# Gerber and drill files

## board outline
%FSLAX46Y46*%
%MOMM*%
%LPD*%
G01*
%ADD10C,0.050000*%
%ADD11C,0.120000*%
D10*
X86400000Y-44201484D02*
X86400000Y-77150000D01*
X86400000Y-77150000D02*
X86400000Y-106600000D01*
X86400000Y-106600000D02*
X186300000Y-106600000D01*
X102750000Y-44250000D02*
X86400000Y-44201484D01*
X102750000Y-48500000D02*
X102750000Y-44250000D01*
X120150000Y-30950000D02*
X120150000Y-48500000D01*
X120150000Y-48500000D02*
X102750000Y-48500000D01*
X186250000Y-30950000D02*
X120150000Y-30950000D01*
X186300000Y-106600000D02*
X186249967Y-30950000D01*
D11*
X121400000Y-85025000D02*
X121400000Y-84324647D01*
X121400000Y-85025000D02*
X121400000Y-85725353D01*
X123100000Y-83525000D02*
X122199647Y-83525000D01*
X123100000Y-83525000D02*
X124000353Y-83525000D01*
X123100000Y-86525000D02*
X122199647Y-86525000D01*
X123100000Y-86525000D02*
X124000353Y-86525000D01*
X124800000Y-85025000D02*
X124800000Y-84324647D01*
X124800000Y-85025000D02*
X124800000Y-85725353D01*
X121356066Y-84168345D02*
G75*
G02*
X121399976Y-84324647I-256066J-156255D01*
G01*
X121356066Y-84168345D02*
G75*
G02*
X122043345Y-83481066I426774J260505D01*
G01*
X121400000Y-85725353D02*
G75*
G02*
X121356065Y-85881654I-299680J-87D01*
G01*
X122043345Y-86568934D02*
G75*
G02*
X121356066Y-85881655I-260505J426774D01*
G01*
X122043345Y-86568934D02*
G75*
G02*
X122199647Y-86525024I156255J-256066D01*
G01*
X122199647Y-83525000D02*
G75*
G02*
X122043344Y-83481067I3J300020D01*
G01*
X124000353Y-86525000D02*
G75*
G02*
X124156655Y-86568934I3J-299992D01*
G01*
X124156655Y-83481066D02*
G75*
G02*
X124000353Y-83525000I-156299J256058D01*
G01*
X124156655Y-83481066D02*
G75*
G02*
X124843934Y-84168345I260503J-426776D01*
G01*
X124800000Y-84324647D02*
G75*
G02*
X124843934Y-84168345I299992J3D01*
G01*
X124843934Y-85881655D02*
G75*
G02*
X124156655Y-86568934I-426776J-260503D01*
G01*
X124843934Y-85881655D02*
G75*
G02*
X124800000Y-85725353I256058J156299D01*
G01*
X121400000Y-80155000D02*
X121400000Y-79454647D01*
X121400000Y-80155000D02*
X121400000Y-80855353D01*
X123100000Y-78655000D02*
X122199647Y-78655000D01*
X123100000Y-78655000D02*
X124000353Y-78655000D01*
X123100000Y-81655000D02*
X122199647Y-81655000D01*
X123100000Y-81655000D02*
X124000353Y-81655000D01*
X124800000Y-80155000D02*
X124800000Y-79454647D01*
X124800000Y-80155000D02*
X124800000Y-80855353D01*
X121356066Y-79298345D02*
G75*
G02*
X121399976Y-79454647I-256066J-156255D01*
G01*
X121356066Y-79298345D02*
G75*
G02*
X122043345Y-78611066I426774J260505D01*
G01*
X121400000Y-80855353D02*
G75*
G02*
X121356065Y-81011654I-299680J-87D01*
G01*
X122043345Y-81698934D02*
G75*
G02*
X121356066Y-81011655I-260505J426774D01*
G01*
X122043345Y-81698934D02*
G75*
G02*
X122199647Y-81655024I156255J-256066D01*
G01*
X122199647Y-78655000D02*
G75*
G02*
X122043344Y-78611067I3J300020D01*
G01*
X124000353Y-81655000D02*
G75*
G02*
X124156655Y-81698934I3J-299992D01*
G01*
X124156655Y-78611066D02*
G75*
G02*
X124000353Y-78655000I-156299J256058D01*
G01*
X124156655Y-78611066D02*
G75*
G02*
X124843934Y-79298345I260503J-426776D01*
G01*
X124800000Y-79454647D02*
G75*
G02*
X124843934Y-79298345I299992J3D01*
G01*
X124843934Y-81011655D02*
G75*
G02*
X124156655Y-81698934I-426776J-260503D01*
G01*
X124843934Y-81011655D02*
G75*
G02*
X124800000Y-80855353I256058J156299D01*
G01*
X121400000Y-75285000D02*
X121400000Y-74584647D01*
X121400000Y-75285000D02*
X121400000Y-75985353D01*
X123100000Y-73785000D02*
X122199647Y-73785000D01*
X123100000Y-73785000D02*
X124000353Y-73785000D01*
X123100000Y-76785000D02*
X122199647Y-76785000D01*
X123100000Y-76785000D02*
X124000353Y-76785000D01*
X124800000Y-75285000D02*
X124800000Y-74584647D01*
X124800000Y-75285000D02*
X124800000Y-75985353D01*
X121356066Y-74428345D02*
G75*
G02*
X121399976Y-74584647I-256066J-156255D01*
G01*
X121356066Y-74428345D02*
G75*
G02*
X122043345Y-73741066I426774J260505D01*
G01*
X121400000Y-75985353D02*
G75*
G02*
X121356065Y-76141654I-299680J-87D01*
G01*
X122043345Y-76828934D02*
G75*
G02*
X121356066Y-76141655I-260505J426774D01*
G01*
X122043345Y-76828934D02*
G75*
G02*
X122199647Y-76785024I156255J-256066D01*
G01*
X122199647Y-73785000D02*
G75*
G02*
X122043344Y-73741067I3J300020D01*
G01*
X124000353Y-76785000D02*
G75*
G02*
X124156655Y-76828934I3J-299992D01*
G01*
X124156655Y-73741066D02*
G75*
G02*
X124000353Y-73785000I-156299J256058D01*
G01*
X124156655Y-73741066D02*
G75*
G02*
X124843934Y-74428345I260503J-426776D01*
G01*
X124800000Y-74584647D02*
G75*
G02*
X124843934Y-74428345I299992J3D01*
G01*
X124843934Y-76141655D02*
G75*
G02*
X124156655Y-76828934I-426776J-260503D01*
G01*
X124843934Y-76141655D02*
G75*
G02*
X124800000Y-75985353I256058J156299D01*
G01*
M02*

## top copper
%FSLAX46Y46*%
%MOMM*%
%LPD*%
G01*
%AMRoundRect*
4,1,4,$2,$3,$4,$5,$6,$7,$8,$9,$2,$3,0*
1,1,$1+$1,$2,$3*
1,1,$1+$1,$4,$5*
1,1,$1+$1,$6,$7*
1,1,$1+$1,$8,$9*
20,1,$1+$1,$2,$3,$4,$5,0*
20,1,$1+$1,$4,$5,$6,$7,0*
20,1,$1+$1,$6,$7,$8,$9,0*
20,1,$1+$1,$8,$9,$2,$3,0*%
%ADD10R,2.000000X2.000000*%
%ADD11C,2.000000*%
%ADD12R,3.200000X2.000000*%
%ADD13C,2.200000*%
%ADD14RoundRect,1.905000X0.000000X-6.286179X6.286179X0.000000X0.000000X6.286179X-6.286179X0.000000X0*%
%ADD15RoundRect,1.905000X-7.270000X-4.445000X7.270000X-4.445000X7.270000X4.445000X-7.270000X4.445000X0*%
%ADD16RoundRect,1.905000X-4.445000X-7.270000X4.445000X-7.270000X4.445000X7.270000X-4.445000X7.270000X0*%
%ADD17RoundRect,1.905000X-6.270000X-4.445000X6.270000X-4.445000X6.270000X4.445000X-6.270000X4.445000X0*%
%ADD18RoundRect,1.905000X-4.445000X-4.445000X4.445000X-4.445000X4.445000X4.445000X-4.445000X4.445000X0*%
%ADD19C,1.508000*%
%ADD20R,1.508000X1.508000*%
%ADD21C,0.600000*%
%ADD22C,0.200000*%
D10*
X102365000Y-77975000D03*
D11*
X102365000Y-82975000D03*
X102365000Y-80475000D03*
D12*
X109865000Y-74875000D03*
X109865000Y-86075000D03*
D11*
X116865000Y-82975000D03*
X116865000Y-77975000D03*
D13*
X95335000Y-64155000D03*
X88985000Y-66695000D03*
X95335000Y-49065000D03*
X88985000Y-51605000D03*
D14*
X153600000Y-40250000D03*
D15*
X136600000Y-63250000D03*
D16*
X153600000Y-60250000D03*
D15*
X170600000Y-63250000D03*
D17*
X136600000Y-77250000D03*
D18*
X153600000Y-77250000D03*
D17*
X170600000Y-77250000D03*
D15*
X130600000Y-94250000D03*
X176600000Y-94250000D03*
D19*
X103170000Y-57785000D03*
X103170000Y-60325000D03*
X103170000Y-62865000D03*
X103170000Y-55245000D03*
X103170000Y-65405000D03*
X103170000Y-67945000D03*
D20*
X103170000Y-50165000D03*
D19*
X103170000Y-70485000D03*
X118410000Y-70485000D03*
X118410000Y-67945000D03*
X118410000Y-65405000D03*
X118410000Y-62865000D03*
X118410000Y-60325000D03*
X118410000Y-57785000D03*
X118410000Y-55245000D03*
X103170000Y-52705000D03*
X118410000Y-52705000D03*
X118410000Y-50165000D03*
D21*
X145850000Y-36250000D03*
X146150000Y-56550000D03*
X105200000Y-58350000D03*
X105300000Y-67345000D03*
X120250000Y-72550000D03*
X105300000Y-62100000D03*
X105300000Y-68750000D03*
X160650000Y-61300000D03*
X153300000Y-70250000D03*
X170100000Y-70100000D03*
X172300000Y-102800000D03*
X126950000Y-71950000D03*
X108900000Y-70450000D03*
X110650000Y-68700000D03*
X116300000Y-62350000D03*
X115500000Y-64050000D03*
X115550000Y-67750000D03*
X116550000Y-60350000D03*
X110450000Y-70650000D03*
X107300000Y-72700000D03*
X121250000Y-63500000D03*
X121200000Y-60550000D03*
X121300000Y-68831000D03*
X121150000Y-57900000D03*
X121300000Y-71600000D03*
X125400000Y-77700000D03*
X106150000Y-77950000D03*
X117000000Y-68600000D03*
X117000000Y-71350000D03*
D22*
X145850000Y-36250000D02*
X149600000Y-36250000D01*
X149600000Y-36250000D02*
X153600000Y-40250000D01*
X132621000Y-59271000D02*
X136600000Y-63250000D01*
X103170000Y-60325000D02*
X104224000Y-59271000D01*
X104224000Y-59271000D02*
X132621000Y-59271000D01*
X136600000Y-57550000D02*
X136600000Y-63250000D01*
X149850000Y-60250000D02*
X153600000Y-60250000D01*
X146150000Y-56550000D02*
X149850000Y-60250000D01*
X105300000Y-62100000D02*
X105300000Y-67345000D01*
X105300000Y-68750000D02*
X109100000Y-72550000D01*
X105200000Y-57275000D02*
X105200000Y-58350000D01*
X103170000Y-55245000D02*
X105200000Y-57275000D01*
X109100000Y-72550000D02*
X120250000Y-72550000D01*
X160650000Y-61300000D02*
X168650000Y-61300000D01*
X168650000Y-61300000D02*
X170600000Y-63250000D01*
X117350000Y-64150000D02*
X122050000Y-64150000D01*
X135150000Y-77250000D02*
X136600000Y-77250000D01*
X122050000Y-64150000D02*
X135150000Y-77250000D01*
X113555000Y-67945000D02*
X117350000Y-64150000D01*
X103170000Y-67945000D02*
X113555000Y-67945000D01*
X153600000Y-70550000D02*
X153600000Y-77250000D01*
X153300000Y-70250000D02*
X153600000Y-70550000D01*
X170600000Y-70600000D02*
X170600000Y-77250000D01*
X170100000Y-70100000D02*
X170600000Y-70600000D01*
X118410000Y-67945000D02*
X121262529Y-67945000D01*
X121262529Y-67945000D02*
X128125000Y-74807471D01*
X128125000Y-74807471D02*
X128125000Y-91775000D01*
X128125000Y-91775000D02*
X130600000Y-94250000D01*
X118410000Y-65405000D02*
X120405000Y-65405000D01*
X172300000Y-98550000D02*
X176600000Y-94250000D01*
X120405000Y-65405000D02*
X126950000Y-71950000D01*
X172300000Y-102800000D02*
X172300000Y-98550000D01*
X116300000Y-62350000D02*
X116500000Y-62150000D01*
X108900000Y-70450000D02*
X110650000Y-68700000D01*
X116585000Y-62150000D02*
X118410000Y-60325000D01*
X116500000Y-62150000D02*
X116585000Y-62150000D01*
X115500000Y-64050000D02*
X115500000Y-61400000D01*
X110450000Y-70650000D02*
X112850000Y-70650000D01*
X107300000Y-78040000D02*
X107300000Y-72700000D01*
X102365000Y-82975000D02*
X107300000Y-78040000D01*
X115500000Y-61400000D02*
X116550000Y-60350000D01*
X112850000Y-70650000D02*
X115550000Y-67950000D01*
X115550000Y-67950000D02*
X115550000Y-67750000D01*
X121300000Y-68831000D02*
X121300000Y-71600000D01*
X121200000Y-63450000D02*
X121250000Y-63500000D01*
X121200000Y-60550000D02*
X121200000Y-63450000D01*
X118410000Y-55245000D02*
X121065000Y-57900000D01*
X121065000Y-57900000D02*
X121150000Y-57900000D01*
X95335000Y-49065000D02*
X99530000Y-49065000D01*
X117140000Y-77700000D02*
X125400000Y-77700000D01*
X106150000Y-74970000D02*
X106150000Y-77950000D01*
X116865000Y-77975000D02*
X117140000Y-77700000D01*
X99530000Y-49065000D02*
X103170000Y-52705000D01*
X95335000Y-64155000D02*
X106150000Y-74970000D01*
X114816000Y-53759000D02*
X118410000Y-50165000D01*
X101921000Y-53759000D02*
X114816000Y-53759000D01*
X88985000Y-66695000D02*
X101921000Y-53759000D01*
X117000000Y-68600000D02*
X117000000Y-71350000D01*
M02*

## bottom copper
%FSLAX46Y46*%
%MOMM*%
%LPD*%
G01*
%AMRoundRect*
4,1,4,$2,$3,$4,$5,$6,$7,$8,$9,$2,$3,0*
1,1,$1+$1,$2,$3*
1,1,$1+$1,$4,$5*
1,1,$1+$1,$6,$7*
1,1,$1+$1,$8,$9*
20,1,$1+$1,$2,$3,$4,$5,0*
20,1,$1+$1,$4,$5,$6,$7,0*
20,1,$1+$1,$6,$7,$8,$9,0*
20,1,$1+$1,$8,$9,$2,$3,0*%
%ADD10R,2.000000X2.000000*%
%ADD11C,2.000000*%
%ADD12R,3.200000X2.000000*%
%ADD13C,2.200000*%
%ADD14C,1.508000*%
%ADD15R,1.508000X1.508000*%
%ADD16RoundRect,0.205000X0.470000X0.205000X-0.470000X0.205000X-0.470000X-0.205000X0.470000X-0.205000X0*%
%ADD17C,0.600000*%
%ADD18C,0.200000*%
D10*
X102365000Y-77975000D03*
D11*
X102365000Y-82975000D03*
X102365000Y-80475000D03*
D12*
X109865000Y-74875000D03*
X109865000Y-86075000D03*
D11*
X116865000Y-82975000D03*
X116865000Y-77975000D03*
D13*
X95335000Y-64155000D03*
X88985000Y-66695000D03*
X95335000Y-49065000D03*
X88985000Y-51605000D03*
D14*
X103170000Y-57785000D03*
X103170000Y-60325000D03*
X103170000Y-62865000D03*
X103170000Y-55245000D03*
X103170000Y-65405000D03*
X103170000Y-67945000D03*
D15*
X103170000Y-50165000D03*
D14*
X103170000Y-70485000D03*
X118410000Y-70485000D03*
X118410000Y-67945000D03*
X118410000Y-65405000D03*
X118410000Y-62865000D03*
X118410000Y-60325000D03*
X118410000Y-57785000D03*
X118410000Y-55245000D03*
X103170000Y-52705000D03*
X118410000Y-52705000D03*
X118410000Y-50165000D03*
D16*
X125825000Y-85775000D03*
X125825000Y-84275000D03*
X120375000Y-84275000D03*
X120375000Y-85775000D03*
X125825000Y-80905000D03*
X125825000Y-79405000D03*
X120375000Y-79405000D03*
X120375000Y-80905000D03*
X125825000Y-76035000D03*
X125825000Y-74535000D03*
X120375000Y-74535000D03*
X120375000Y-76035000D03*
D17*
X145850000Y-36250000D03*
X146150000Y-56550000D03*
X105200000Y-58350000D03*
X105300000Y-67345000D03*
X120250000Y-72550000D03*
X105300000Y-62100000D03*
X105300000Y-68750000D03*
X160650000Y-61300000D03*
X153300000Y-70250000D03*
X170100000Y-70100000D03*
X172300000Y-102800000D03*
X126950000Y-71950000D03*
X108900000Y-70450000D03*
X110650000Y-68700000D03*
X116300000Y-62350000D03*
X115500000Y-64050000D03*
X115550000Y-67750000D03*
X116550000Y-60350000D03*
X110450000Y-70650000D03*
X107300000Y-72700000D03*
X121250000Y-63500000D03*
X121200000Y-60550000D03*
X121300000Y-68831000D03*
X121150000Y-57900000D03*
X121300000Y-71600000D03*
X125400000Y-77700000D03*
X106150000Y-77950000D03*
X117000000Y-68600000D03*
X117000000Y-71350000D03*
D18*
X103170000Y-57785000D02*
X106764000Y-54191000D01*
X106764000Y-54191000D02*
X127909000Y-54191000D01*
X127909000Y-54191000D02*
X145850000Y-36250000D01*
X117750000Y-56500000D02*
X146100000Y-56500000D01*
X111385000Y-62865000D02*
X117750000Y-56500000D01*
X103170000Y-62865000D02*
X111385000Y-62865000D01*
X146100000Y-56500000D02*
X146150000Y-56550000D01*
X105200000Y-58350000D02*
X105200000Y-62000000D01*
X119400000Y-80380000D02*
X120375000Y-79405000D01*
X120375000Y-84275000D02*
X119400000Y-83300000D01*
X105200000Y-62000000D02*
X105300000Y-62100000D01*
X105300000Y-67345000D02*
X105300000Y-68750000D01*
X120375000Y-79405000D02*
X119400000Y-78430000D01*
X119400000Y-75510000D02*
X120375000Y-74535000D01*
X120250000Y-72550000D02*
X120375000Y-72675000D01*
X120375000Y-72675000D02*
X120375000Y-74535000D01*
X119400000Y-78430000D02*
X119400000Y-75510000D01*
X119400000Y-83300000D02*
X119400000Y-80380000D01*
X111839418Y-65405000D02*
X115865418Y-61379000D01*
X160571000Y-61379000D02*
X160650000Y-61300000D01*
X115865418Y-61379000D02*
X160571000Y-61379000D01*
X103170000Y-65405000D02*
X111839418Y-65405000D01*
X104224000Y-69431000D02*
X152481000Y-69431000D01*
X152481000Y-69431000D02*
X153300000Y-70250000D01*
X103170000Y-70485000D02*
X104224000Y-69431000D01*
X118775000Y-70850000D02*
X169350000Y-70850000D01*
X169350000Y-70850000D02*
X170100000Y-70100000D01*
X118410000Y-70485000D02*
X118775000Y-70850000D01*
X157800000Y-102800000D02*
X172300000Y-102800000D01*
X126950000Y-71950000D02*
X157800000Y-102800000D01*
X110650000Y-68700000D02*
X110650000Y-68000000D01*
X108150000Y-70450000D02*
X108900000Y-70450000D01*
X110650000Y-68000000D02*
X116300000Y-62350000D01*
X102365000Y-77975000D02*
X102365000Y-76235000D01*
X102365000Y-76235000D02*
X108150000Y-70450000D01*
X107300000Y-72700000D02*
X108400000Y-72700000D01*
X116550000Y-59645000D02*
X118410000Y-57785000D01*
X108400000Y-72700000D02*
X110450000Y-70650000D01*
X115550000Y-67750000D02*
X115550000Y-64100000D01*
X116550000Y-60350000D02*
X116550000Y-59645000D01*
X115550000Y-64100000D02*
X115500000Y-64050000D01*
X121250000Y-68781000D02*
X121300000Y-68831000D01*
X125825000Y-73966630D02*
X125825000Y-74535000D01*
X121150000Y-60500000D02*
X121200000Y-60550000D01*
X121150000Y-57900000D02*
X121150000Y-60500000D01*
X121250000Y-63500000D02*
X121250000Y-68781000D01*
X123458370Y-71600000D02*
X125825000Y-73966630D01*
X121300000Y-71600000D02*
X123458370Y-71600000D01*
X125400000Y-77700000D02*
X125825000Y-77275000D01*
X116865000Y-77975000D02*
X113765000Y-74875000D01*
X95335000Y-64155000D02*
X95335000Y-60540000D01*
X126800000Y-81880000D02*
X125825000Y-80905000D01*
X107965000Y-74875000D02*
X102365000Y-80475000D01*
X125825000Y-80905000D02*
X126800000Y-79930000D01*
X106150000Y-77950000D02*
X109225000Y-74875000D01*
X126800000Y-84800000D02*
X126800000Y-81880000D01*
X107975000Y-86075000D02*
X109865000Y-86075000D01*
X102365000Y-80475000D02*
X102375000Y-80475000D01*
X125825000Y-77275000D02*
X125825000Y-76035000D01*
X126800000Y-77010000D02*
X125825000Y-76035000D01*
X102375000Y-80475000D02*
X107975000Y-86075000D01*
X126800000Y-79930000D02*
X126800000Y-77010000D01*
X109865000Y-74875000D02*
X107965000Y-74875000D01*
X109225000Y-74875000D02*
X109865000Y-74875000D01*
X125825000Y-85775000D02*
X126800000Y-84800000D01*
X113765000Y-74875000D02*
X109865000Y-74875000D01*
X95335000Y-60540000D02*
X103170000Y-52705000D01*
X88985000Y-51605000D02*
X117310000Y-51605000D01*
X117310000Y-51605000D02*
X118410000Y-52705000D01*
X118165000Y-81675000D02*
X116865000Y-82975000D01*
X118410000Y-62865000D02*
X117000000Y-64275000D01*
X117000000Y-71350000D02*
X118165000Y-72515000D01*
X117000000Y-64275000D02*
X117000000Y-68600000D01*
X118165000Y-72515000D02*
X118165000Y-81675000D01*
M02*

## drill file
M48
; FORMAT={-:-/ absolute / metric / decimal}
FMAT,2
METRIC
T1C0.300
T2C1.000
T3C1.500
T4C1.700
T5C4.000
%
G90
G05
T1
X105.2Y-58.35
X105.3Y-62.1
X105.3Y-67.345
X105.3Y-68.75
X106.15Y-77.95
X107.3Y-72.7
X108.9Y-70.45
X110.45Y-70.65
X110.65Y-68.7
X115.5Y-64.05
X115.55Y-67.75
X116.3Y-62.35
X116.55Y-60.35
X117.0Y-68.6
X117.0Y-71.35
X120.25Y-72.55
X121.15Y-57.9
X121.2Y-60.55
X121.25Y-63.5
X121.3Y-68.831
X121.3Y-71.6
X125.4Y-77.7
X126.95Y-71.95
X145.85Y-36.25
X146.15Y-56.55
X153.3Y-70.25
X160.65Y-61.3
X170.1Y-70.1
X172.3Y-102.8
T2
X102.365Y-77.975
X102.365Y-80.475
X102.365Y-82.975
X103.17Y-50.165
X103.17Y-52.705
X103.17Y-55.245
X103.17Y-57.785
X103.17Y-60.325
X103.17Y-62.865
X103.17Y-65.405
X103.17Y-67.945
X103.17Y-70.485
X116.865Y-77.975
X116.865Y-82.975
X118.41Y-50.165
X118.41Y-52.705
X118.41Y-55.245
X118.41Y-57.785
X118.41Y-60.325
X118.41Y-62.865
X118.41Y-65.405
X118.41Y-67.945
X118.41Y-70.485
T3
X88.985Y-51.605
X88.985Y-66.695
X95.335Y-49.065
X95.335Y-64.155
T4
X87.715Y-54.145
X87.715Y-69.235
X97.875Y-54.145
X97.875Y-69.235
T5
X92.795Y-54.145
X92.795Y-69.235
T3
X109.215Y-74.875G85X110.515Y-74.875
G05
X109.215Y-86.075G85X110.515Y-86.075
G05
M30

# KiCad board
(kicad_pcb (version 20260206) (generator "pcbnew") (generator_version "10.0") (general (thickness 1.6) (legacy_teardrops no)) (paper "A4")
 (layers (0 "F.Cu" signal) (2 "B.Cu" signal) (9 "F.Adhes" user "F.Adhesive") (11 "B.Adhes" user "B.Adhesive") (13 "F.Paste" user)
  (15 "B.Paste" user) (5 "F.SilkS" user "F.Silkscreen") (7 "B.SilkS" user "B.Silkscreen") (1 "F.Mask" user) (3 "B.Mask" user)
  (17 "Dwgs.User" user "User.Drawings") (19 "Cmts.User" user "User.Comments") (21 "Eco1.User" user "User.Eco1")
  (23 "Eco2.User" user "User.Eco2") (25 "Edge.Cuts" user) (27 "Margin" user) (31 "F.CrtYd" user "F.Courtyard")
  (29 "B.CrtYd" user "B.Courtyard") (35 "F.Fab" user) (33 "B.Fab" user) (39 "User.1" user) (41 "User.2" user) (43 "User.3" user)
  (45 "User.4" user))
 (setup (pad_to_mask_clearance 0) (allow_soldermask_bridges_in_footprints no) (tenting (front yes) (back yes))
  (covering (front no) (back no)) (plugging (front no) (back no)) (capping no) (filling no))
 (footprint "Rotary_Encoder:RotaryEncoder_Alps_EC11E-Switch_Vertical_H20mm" (layer "F.Cu") (at 102.365 77.975)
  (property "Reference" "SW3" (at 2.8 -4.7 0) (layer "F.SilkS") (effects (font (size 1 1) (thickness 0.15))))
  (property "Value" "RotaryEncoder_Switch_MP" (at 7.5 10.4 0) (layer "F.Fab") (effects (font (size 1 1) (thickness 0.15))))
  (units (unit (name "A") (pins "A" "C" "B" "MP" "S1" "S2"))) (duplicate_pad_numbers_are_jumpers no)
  (pad "A" thru_hole rect (at 0 0) (size 2 2) (drill 1) (layers "*.Cu" "*.Mask") (remove_unused_layers no) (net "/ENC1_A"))
  (pad "B" thru_hole circle (at 0 5) (size 2 2) (drill 1) (layers "*.Cu" "*.Mask") (remove_unused_layers no) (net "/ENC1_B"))
  (pad "C" thru_hole circle (at 0 2.5) (size 2 2) (drill 1) (layers "*.Cu" "*.Mask") (remove_unused_layers no) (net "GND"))
  (pad "MP" thru_hole rect (at 7.5 -3.1) (size 3.2 2) (drill oval 2.8 1.5) (layers "*.Cu" "*.Mask") (remove_unused_layers no) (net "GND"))
  (pad "MP" thru_hole rect (at 7.5 8.1) (size 3.2 2) (drill oval 2.8 1.5) (layers "*.Cu" "*.Mask") (remove_unused_layers no) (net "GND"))
  (pad "S1" thru_hole circle (at 14.5 5) (size 2 2) (drill 1) (layers "*.Cu" "*.Mask") (remove_unused_layers no) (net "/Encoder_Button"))
  (pad "S2" thru_hole circle (at 14.5 0) (size 2 2) (drill 1) (layers "*.Cu" "*.Mask") (remove_unused_layers no) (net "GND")))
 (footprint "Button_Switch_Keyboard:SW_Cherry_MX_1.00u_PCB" (layer "F.Cu") (at 95.335 64.155)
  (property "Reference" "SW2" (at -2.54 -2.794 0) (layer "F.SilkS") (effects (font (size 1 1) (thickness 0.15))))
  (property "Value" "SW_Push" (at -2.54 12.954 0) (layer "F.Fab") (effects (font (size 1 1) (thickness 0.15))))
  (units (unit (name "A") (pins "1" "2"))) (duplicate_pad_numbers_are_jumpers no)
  (pad "" np_thru_hole circle (at -7.62 5.08) (size 1.7 1.7) (drill 1.7) (layers "*.Cu" "*.Mask"))
  (pad "" np_thru_hole circle (at -2.54 5.08) (size 4 4) (drill 4) (layers "*.Cu" "*.Mask"))
  (pad "" np_thru_hole circle (at 2.54 5.08) (size 1.7 1.7) (drill 1.7) (layers "*.Cu" "*.Mask"))
  (pad "1" thru_hole circle (at 0 0) (size 2.2 2.2) (drill 1.5) (layers "*.Cu" "*.Mask") (remove_unused_layers no) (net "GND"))
  (pad "2" thru_hole circle (at -6.35 2.54) (size 2.2 2.2) (drill 1.5) (layers "*.Cu" "*.Mask") (remove_unused_layers no) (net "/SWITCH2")))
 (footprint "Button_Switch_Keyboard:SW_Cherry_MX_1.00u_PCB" (layer "F.Cu") (at 95.335 49.065)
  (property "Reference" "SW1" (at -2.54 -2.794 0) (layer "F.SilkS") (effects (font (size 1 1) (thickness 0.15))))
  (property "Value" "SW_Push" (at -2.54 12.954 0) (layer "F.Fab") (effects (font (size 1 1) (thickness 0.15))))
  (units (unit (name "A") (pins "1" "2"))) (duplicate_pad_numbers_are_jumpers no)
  (pad "" np_thru_hole circle (at -7.62 5.08) (size 1.7 1.7) (drill 1.7) (layers "*.Cu" "*.Mask"))
  (pad "" np_thru_hole circle (at -2.54 5.08) (size 4 4) (drill 4) (layers "*.Cu" "*.Mask"))
  (pad "" np_thru_hole circle (at 2.54 5.08) (size 1.7 1.7) (drill 1.7) (layers "*.Cu" "*.Mask"))
  (pad "1" thru_hole circle (at 0 0) (size 2.2 2.2) (drill 1.5) (layers "*.Cu" "*.Mask") (remove_unused_layers no) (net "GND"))
  (pad "2" thru_hole circle (at -6.35 2.54) (size 2.2 2.2) (drill 1.5) (layers "*.Cu" "*.Mask") (remove_unused_layers no) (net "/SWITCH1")))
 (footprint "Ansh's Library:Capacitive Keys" (layer "F.Cu") (at 159.6 36.25)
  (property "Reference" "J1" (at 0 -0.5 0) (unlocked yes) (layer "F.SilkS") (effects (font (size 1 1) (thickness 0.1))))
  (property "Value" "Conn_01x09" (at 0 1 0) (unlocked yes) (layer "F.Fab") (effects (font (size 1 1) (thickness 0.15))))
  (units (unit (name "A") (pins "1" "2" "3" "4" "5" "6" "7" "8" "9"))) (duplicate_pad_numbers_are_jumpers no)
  (pad "1" smd roundrect (at -6 4 45) (size 12.7 12.7) (layers "F.Cu" "F.Mask") (roundrect_rratio 0.15) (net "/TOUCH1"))
  (pad "2" smd roundrect (at -23 27) (size 18.35 12.7) (layers "F.Cu" "F.Mask") (roundrect_rratio 0.15) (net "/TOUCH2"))
  (pad "3" smd roundrect (at -6 24) (size 12.7 18.35) (layers "F.Cu" "F.Mask") (roundrect_rratio 0.15) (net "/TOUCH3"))
  (pad "4" smd roundrect (at 11 27) (size 18.35 12.7) (layers "F.Cu" "F.Mask") (roundrect_rratio 0.15) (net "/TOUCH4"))
  (pad "5" smd roundrect (at -23 41) (size 16.35 12.7) (layers "F.Cu" "F.Mask") (roundrect_rratio 0.15) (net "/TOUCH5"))
  (pad "6" smd roundrect (at -6 41) (size 12.7 12.7) (layers "F.Cu" "F.Mask") (roundrect_rratio 0.15) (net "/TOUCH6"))
  (pad "7" smd roundrect (at 11 41) (size 16.35 12.7) (layers "F.Cu" "F.Mask") (roundrect_rratio 0.15) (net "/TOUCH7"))
  (pad "8" smd roundrect (at -29 58) (size 18.35 12.7) (layers "F.Cu" "F.Mask") (roundrect_rratio 0.15) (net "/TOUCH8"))
  (pad "9" smd roundrect (at 17 58) (size 18.35 12.7) (layers "F.Cu" "F.Mask") (roundrect_rratio 0.15) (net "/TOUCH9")))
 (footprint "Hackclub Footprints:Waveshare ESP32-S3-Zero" (layer "F.Cu") (at 110.79 60.325)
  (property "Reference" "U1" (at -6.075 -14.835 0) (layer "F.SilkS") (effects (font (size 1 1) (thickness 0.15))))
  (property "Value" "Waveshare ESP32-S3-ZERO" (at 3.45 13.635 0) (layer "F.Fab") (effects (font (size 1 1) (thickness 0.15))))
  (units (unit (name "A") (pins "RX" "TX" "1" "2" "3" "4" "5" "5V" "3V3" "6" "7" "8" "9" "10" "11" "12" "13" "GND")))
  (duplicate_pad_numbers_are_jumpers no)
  (pad "1" thru_hole circle (at -7.62 -2.54) (size 1.508 1.508) (drill 1) (layers "*.Cu" "*.Mask") (remove_unused_layers no) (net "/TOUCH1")
   (solder_mask_margin 0.102))
  (pad "2" thru_hole circle (at -7.62 0) (size 1.508 1.508) (drill 1) (layers "*.Cu" "*.Mask") (remove_unused_layers no) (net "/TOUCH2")
   (solder_mask_margin 0.102))
  (pad "3" thru_hole circle (at -7.62 2.54) (size 1.508 1.508) (drill 1) (layers "*.Cu" "*.Mask") (remove_unused_layers no) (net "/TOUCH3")
   (solder_mask_margin 0.102))
  (pad "3V3" thru_hole circle (at -7.62 -5.08) (size 1.508 1.508) (drill 1) (layers "*.Cu" "*.Mask") (remove_unused_layers no) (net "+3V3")
   (solder_mask_margin 0.102))
  (pad "4" thru_hole circle (at -7.62 5.08) (size 1.508 1.508) (drill 1) (layers "*.Cu" "*.Mask") (remove_unused_layers no) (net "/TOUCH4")
   (solder_mask_margin 0.102))
  (pad "5" thru_hole circle (at -7.62 7.62) (size 1.508 1.508) (drill 1) (layers "*.Cu" "*.Mask") (remove_unused_layers no) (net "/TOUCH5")
   (solder_mask_margin 0.102))
  (pad "5V" thru_hole rect (at -7.62 -10.16) (size 1.508 1.508) (drill 1) (layers "*.Cu" "*.Mask") (remove_unused_layers no) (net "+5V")
   (solder_mask_margin 0.102))
  (pad "6" thru_hole circle (at -7.62 10.16) (size 1.508 1.508) (drill 1) (layers "*.Cu" "*.Mask") (remove_unused_layers no) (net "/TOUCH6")
   (solder_mask_margin 0.102))
  (pad "7" thru_hole circle (at 7.62 10.16) (size 1.508 1.508) (drill 1) (layers "*.Cu" "*.Mask") (remove_unused_layers no) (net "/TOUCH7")
   (solder_mask_margin 0.102))
  (pad "8" thru_hole circle (at 7.62 7.62) (size 1.508 1.508) (drill 1) (layers "*.Cu" "*.Mask") (remove_unused_layers no) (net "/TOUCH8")
   (solder_mask_margin 0.102))
  (pad "9" thru_hole circle (at 7.62 5.08) (size 1.508 1.508) (drill 1) (layers "*.Cu" "*.Mask") (remove_unused_layers no) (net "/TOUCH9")
   (solder_mask_margin 0.102))
  (pad "10" thru_hole circle (at 7.62 2.54) (size 1.508 1.508) (drill 1) (layers "*.Cu" "*.Mask") (remove_unused_layers no)
   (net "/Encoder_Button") (solder_mask_margin 0.102))
  (pad "11" thru_hole circle (at 7.62 0) (size 1.508 1.508) (drill 1) (layers "*.Cu" "*.Mask") (remove_unused_layers no) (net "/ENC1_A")
   (solder_mask_margin 0.102))
  (pad "12" thru_hole circle (at 7.62 -2.54) (size 1.508 1.508) (drill 1) (layers "*.Cu" "*.Mask") (remove_unused_layers no) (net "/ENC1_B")
   (solder_mask_margin 0.102))
  (pad "13" thru_hole circle (at 7.62 -5.08) (size 1.508 1.508) (drill 1) (layers "*.Cu" "*.Mask") (remove_unused_layers no) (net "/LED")
   (solder_mask_margin 0.102))
  (pad "GND" thru_hole circle (at -7.62 -7.62) (size 1.508 1.508) (drill 1) (layers "*.Cu" "*.Mask") (remove_unused_layers no) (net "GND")
   (solder_mask_margin 0.102))
  (pad "RX" thru_hole circle (at 7.62 -7.62) (size 1.508 1.508) (drill 1) (layers "*.Cu" "*.Mask") (remove_unused_layers no)
   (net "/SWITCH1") (solder_mask_margin 0.102))
  (pad "TX" thru_hole circle (at 7.62 -10.16) (size 1.508 1.508) (drill 1) (layers "*.Cu" "*.Mask") (remove_unused_layers no)
   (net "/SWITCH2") (solder_mask_margin 0.102)))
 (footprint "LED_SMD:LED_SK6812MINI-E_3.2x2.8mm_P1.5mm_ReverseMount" (layer "B.Cu") (at 123.1 85.025 180)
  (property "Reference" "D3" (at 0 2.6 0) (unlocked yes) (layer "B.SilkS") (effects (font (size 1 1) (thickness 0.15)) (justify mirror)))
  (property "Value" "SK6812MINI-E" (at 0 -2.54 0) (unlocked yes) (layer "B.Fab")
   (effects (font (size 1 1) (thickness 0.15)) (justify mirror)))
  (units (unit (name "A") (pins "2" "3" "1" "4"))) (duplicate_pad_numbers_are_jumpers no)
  (fp_line (start 1.7 0) (end 1.7 0.700353) (stroke (width 0.12) (type solid)) (layer "Edge.Cuts"))
  (fp_line (start 1.7 0) (end 1.7 -0.700353) (stroke (width 0.12) (type solid)) (layer "Edge.Cuts"))
  (fp_line (start 0 1.5) (end 0.900353 1.5) (stroke (width 0.12) (type solid)) (layer "Edge.Cuts"))
  (fp_line (start 0 1.5) (end -0.900353 1.5) (stroke (width 0.12) (type solid)) (layer "Edge.Cuts"))
  (fp_line (start 0 -1.5) (end 0.900353 -1.5) (stroke (width 0.12) (type solid)) (layer "Edge.Cuts"))
  (fp_line (start 0 -1.5) (end -0.900353 -1.5) (stroke (width 0.12) (type solid)) (layer "Edge.Cuts"))
  (fp_line (start -1.7 0) (end -1.7 0.700353) (stroke (width 0.12) (type solid)) (layer "Edge.Cuts"))
  (fp_line (start -1.7 0) (end -1.7 -0.700353) (stroke (width 0.12) (type solid)) (layer "Edge.Cuts"))
  (fp_arc (start 1.743934 0.856655) (mid 1.711191 0.781533) (end 1.7 0.700353) (stroke (width 0.12) (type solid)) (layer "Edge.Cuts"))
  (fp_arc (start 1.743934 0.856655) (mid 1.670713 1.470713) (end 1.056655 1.543934) (stroke (width 0.12) (type solid)) (layer "Edge.Cuts"))
  (fp_arc (start 1.7 -0.700353) (mid 1.711181 -0.781538) (end 1.743934 -0.856655) (stroke (width 0.12) (type solid)) (layer "Edge.Cuts"))
  (fp_arc (start 1.056655 -1.543934) (mid 1.670711 -1.470711) (end 1.743934 -0.856655) (stroke (width 0.12) (type solid))
   (layer "Edge.Cuts"))
  (fp_arc (start 1.056655 -1.543934) (mid 0.981533 -1.511191) (end 0.900353 -1.5) (stroke (width 0.12) (type solid)) (layer "Edge.Cuts"))
  (fp_arc (start 0.900353 1.5) (mid 0.981532 1.511193) (end 1.056655 1.543934) (stroke (width 0.12) (type solid)) (layer "Edge.Cuts"))
  (fp_arc (start -0.900353 -1.5) (mid -0.981533 -1.511192) (end -1.056655 -1.543934) (stroke (width 0.12) (type solid)) (layer "Edge.Cuts"))
  (fp_arc (start -1.056655 1.543934) (mid -0.981533 1.511192) (end -0.900353 1.5) (stroke (width 0.12) (type solid)) (layer "Edge.Cuts"))
  (fp_arc (start -1.056655 1.543934) (mid -1.670711 1.470711) (end -1.743934 0.856655) (stroke (width 0.12) (type solid))
   (layer "Edge.Cuts"))
  (fp_arc (start -1.7 0.700353) (mid -1.711192 0.781533) (end -1.743934 0.856655) (stroke (width 0.12) (type solid)) (layer "Edge.Cuts"))
  (fp_arc (start -1.743934 -0.856655) (mid -1.670711 -1.470711) (end -1.056655 -1.543934) (stroke (width 0.12) (type solid))
   (layer "Edge.Cuts"))
  (fp_arc (start -1.743934 -0.856655) (mid -1.711192 -0.781533) (end -1.7 -0.700353) (stroke (width 0.12) (type solid)) (layer "Edge.Cuts"))
  (pad "1" smd roundrect (at -2.725 -0.75 180) (size 1.35 0.82) (layers "B.Cu" "B.Mask" "B.Paste") (roundrect_rratio 0.25) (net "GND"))
  (pad "2" smd roundrect (at -2.725 0.75 180) (size 1.35 0.82) (layers "B.Cu" "B.Mask" "B.Paste") (roundrect_rratio 0.25)
   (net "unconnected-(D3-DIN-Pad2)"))
  (pad "3" smd roundrect (at 2.725 0.75 180) (size 1.35 0.82) (layers "B.Cu" "B.Mask" "B.Paste") (roundrect_rratio 0.25) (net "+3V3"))
  (pad "4" smd roundrect (at 2.725 -0.75 180) (size 1.35 0.82) (layers "B.Cu" "B.Mask" "B.Paste") (roundrect_rratio 0.25)
   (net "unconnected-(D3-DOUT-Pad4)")))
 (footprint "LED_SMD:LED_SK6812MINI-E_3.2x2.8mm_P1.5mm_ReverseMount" (layer "B.Cu") (at 123.1 80.155 180)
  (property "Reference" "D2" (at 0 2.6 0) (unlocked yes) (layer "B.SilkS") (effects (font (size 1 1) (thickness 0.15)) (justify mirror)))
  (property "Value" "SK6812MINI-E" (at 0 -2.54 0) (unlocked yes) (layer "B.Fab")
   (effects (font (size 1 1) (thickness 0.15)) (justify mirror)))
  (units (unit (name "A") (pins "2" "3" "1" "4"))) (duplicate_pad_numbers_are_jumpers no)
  (fp_line (start 1.7 0) (end 1.7 0.700353) (stroke (width 0.12) (type solid)) (layer "Edge.Cuts"))
  (fp_line (start 1.7 0) (end 1.7 -0.700353) (stroke (width 0.12) (type solid)) (layer "Edge.Cuts"))
  (fp_line (start 0 1.5) (end 0.900353 1.5) (stroke (width 0.12) (type solid)) (layer "Edge.Cuts"))
  (fp_line (start 0 1.5) (end -0.900353 1.5) (stroke (width 0.12) (type solid)) (layer "Edge.Cuts"))
  (fp_line (start 0 -1.5) (end 0.900353 -1.5) (stroke (width 0.12) (type solid)) (layer "Edge.Cuts"))
  (fp_line (start 0 -1.5) (end -0.900353 -1.5) (stroke (width 0.12) (type solid)) (layer "Edge.Cuts"))
  (fp_line (start -1.7 0) (end -1.7 0.700353) (stroke (width 0.12) (type solid)) (layer "Edge.Cuts"))
  (fp_line (start -1.7 0) (end -1.7 -0.700353) (stroke (width 0.12) (type solid)) (layer "Edge.Cuts"))
  (fp_arc (start 1.743934 0.856655) (mid 1.711191 0.781533) (end 1.7 0.700353) (stroke (width 0.12) (type solid)) (layer "Edge.Cuts"))
  (fp_arc (start 1.743934 0.856655) (mid 1.670713 1.470713) (end 1.056655 1.543934) (stroke (width 0.12) (type solid)) (layer "Edge.Cuts"))
  (fp_arc (start 1.7 -0.700353) (mid 1.711181 -0.781538) (end 1.743934 -0.856655) (stroke (width 0.12) (type solid)) (layer "Edge.Cuts"))
  (fp_arc (start 1.056655 -1.543934) (mid 1.670711 -1.470711) (end 1.743934 -0.856655) (stroke (width 0.12) (type solid))
   (layer "Edge.Cuts"))
  (fp_arc (start 1.056655 -1.543934) (mid 0.981533 -1.511191) (end 0.900353 -1.5) (stroke (width 0.12) (type solid)) (layer "Edge.Cuts"))
  (fp_arc (start 0.900353 1.5) (mid 0.981532 1.511193) (end 1.056655 1.543934) (stroke (width 0.12) (type solid)) (layer "Edge.Cuts"))
  (fp_arc (start -0.900353 -1.5) (mid -0.981533 -1.511192) (end -1.056655 -1.543934) (stroke (width 0.12) (type solid)) (layer "Edge.Cuts"))
  (fp_arc (start -1.056655 1.543934) (mid -0.981533 1.511192) (end -0.900353 1.5) (stroke (width 0.12) (type solid)) (layer "Edge.Cuts"))
  (fp_arc (start -1.056655 1.543934) (mid -1.670711 1.470711) (end -1.743934 0.856655) (stroke (width 0.12) (type solid))
   (layer "Edge.Cuts"))
  (fp_arc (start -1.7 0.700353) (mid -1.711192 0.781533) (end -1.743934 0.856655) (stroke (width 0.12) (type solid)) (layer "Edge.Cuts"))
  (fp_arc (start -1.743934 -0.856655) (mid -1.670711 -1.470711) (end -1.056655 -1.543934) (stroke (width 0.12) (type solid))
   (layer "Edge.Cuts"))
  (fp_arc (start -1.743934 -0.856655) (mid -1.711192 -0.781533) (end -1.7 -0.700353) (stroke (width 0.12) (type solid)) (layer "Edge.Cuts"))
  (pad "1" smd roundrect (at -2.725 -0.75 180) (size 1.35 0.82) (layers "B.Cu" "B.Mask" "B.Paste") (roundrect_rratio 0.25) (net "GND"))
  (pad "2" smd roundrect (at -2.725 0.75 180) (size 1.35 0.82) (layers "B.Cu" "B.Mask" "B.Paste") (roundrect_rratio 0.25)
   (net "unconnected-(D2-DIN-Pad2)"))
  (pad "3" smd roundrect (at 2.725 0.75 180) (size 1.35 0.82) (layers "B.Cu" "B.Mask" "B.Paste") (roundrect_rratio 0.25) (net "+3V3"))
  (pad "4" smd roundrect (at 2.725 -0.75 180) (size 1.35 0.82) (layers "B.Cu" "B.Mask" "B.Paste") (roundrect_rratio 0.25)
   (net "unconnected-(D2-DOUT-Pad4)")))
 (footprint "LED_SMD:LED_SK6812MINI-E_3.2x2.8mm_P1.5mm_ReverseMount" (layer "B.Cu") (at 123.1 75.285 180)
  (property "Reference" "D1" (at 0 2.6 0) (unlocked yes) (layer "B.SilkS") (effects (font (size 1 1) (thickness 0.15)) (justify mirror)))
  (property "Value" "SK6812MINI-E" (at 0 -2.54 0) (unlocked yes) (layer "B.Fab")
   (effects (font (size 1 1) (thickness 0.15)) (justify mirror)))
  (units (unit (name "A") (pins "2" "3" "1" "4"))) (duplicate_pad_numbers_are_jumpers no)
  (fp_line (start 1.7 0) (end 1.7 0.700353) (stroke (width 0.12) (type solid)) (layer "Edge.Cuts"))
  (fp_line (start 1.7 0) (end 1.7 -0.700353) (stroke (width 0.12) (type solid)) (layer "Edge.Cuts"))
  (fp_line (start 0 1.5) (end 0.900353 1.5) (stroke (width 0.12) (type solid)) (layer "Edge.Cuts"))
  (fp_line (start 0 1.5) (end -0.900353 1.5) (stroke (width 0.12) (type solid)) (layer "Edge.Cuts"))
  (fp_line (start 0 -1.5) (end 0.900353 -1.5) (stroke (width 0.12) (type solid)) (layer "Edge.Cuts"))
  (fp_line (start 0 -1.5) (end -0.900353 -1.5) (stroke (width 0.12) (type solid)) (layer "Edge.Cuts"))
  (fp_line (start -1.7 0) (end -1.7 0.700353) (stroke (width 0.12) (type solid)) (layer "Edge.Cuts"))
  (fp_line (start -1.7 0) (end -1.7 -0.700353) (stroke (width 0.12) (type solid)) (layer "Edge.Cuts"))
  (fp_arc (start 1.743934 0.856655) (mid 1.711191 0.781533) (end 1.7 0.700353) (stroke (width 0.12) (type solid)) (layer "Edge.Cuts"))
  (fp_arc (start 1.743934 0.856655) (mid 1.670713 1.470713) (end 1.056655 1.543934) (stroke (width 0.12) (type solid)) (layer "Edge.Cuts"))
  (fp_arc (start 1.7 -0.700353) (mid 1.711181 -0.781538) (end 1.743934 -0.856655) (stroke (width 0.12) (type solid)) (layer "Edge.Cuts"))
  (fp_arc (start 1.056655 -1.543934) (mid 1.670711 -1.470711) (end 1.743934 -0.856655) (stroke (width 0.12) (type solid))
   (layer "Edge.Cuts"))
  (fp_arc (start 1.056655 -1.543934) (mid 0.981533 -1.511191) (end 0.900353 -1.5) (stroke (width 0.12) (type solid)) (layer "Edge.Cuts"))
  (fp_arc (start 0.900353 1.5) (mid 0.981532 1.511193) (end 1.056655 1.543934) (stroke (width 0.12) (type solid)) (layer "Edge.Cuts"))
  (fp_arc (start -0.900353 -1.5) (mid -0.981533 -1.511192) (end -1.056655 -1.543934) (stroke (width 0.12) (type solid)) (layer "Edge.Cuts"))
  (fp_arc (start -1.056655 1.543934) (mid -0.981533 1.511192) (end -0.900353 1.5) (stroke (width 0.12) (type solid)) (layer "Edge.Cuts"))
  (fp_arc (start -1.056655 1.543934) (mid -1.670711 1.470711) (end -1.743934 0.856655) (stroke (width 0.12) (type solid))
   (layer "Edge.Cuts"))
  (fp_arc (start -1.7 0.700353) (mid -1.711192 0.781533) (end -1.743934 0.856655) (stroke (width 0.12) (type solid)) (layer "Edge.Cuts"))
  (fp_arc (start -1.743934 -0.856655) (mid -1.670711 -1.470711) (end -1.056655 -1.543934) (stroke (width 0.12) (type solid))
   (layer "Edge.Cuts"))
  (fp_arc (start -1.743934 -0.856655) (mid -1.711192 -0.781533) (end -1.7 -0.700353) (stroke (width 0.12) (type solid)) (layer "Edge.Cuts"))
  (pad "1" smd roundrect (at -2.725 -0.75 180) (size 1.35 0.82) (layers "B.Cu" "B.Mask" "B.Paste") (roundrect_rratio 0.25) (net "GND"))
  (pad "2" smd roundrect (at -2.725 0.75 180) (size 1.35 0.82) (layers "B.Cu" "B.Mask" "B.Paste") (roundrect_rratio 0.25) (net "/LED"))
  (pad "3" smd roundrect (at 2.725 0.75 180) (size 1.35 0.82) (layers "B.Cu" "B.Mask" "B.Paste") (roundrect_rratio 0.25) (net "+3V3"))
  (pad "4" smd roundrect (at 2.725 -0.75 180) (size 1.35 0.82) (layers "B.Cu" "B.Mask" "B.Paste") (roundrect_rratio 0.25)
   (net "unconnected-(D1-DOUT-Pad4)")))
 (gr_line (start 86.4 44.201484) (end 86.4 77.15) (stroke (width 0.05) (type default)) (layer "Edge.Cuts"))
 (gr_line (start 86.4 77.15) (end 86.4 106.6) (stroke (width 0.05) (type default)) (layer "Edge.Cuts"))
 (gr_line (start 86.4 106.6) (end 186.3 106.6) (stroke (width 0.05) (type default)) (layer "Edge.Cuts"))
 (gr_line (start 102.75 44.25) (end 86.4 44.201484) (stroke (width 0.05) (type default)) (layer "Edge.Cuts"))
 (gr_line (start 102.75 48.5) (end 102.75 44.25) (stroke (width 0.05) (type default)) (layer "Edge.Cuts"))
 (gr_line (start 120.15 30.95) (end 120.15 48.5) (stroke (width 0.05) (type default)) (layer "Edge.Cuts"))
 (gr_line (start 120.15 48.5) (end 102.75 48.5) (stroke (width 0.05) (type default)) (layer "Edge.Cuts"))
 (gr_line (start 186.25 30.95) (end 120.15 30.95) (stroke (width 0.05) (type default)) (layer "Edge.Cuts"))
 (gr_line (start 186.3 106.6) (end 186.249967 30.95) (stroke (width 0.05) (type default)) (layer "Edge.Cuts"))
 (segment (start 145.85 36.25) (end 149.6 36.25) (width 0.2) (layer "F.Cu") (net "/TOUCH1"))
 (segment (start 149.6 36.25) (end 153.6 40.25) (width 0.2) (layer "F.Cu") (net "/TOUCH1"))
 (via (at 145.85 36.25) (size 0.6) (drill 0.3) (layers "F.Cu" "B.Cu") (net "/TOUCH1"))
 (segment (start 103.17 57.785) (end 106.764 54.191) (width 0.2) (layer "B.Cu") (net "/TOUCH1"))
 (segment (start 106.764 54.191) (end 127.909 54.191) (width 0.2) (layer "B.Cu") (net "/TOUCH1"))
 (segment (start 127.909 54.191) (end 145.85 36.25) (width 0.2) (layer "B.Cu") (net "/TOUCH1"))
 (segment (start 132.621 59.271) (end 136.6 63.25) (width 0.2) (layer "F.Cu") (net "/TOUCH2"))
 (segment (start 103.17 60.325) (end 104.224 59.271) (width 0.2) (layer "F.Cu") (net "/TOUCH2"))
 (segment (start 104.224 59.271) (end 132.621 59.271) (width 0.2) (layer "F.Cu") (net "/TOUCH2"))
 (segment (start 136.6 57.55) (end 136.6 63.25) (width 0.2) (layer "F.Cu") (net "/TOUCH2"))
 (segment (start 149.85 60.25) (end 153.6 60.25) (width 0.2) (layer "F.Cu") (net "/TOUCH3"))
 (segment (start 146.15 56.55) (end 149.85 60.25) (width 0.2) (layer "F.Cu") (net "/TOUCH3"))
 (via (at 146.15 56.55) (size 0.6) (drill 0.3) (layers "F.Cu" "B.Cu") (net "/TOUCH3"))
 (segment (start 117.75 56.5) (end 146.1 56.5) (width 0.2) (layer "B.Cu") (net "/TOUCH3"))
 (segment (start 111.385 62.865) (end 117.75 56.5) (width 0.2) (layer "B.Cu") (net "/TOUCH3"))
 (segment (start 103.17 62.865) (end 111.385 62.865) (width 0.2) (layer "B.Cu") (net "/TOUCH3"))
 (segment (start 146.1 56.5) (end 146.15 56.55) (width 0.2) (layer "B.Cu") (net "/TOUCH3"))
 (segment (start 105.3 62.1) (end 105.3 67.345) (width 0.2) (layer "F.Cu") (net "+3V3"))
 (segment (start 105.3 68.75) (end 109.1 72.55) (width 0.2) (layer "F.Cu") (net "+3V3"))
 (segment (start 105.2 57.275) (end 105.2 58.35) (width 0.2) (layer "F.Cu") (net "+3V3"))
 (segment (start 103.17 55.245) (end 105.2 57.275) (width 0.2) (layer "F.Cu") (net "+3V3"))
 (segment (start 109.1 72.55) (end 120.25 72.55) (width 0.2) (layer "F.Cu") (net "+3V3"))
 (via (at 105.2 58.35) (size 0.6) (drill 0.3) (layers "F.Cu" "B.Cu") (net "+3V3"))
 (via (at 105.3 67.345) (size 0.6) (drill 0.3) (layers "F.Cu" "B.Cu") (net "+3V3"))
 (via (at 120.25 72.55) (size 0.6) (drill 0.3) (layers "F.Cu" "B.Cu") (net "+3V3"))
 (via (at 105.3 62.1) (size 0.6) (drill 0.3) (layers "F.Cu" "B.Cu") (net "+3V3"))
 (via (at 105.3 68.75) (size 0.6) (drill 0.3) (layers "F.Cu" "B.Cu") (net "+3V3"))
 (segment (start 105.2 58.35) (end 105.2 62) (width 0.2) (layer "B.Cu") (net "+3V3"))
 (segment (start 119.4 80.38) (end 120.375 79.405) (width 0.2) (layer "B.Cu") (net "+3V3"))
 (segment (start 120.375 84.275) (end 119.4 83.3) (width 0.2) (layer "B.Cu") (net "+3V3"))
 (segment (start 105.2 62) (end 105.3 62.1) (width 0.2) (layer "B.Cu") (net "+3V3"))
 (segment (start 105.3 67.345) (end 105.3 68.75) (width 0.2) (layer "B.Cu") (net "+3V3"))
 (segment (start 120.375 79.405) (end 119.4 78.43) (width 0.2) (layer "B.Cu") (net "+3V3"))
 (segment (start 119.4 75.51) (end 120.375 74.535) (width 0.2) (layer "B.Cu") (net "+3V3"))
 (segment (start 120.25 72.55) (end 120.375 72.675) (width 0.2) (layer "B.Cu") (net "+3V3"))
 (segment (start 120.375 72.675) (end 120.375 74.535) (width 0.2) (layer "B.Cu") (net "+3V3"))
 (segment (start 119.4 78.43) (end 119.4 75.51) (width 0.2) (layer "B.Cu") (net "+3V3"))
 (segment (start 119.4 83.3) (end 119.4 80.38) (width 0.2) (layer "B.Cu") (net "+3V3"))
 (segment (start 160.65 61.3) (end 168.65 61.3) (width 0.2) (layer "F.Cu") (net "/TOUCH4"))
 (segment (start 168.65 61.3) (end 170.6 63.25) (width 0.2) (layer "F.Cu") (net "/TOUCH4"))
 (via (at 160.65 61.3) (size 0.6) (drill 0.3) (layers "F.Cu" "B.Cu") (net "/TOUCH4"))
 (segment (start 111.839418 65.405) (end 115.865418 61.379) (width 0.2) (layer "B.Cu") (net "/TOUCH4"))
 (segment (start 160.571 61.379) (end 160.65 61.3) (width 0.2) (layer "B.Cu") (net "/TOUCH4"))
 (segment (start 115.865418 61.379) (end 160.571 61.379) (width 0.2) (layer "B.Cu") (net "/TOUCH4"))
 (segment (start 103.17 65.405) (end 111.839418 65.405) (width 0.2) (layer "B.Cu") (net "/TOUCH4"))
 (segment (start 117.35 64.15) (end 122.05 64.15) (width 0.2) (layer "F.Cu") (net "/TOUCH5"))
 (segment (start 135.15 77.25) (end 136.6 77.25) (width 0.2) (layer "F.Cu") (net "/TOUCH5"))
 (segment (start 122.05 64.15) (end 135.15 77.25) (width 0.2) (layer "F.Cu") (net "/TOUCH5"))
 (segment (start 113.555 67.945) (end 117.35 64.15) (width 0.2) (layer "F.Cu") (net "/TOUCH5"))
 (segment (start 103.17 67.945) (end 113.555 67.945) (width 0.2) (layer "F.Cu") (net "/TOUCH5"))
 (segment (start 153.6 70.55) (end 153.6 77.25) (width 0.2) (layer "F.Cu") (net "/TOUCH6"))
 (segment (start 153.3 70.25) (end 153.6 70.55) (width 0.2) (layer "F.Cu") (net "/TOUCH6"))
 (via (at 153.3 70.25) (size 0.6) (drill 0.3) (layers "F.Cu" "B.Cu") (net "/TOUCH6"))
 (segment (start 104.224 69.431) (end 152.481 69.431) (width 0.2) (layer "B.Cu") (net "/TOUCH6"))
 (segment (start 152.481 69.431) (end 153.3 70.25) (width 0.2) (layer "B.Cu") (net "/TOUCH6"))
 (segment (start 103.17 70.485) (end 104.224 69.431) (width 0.2) (layer "B.Cu") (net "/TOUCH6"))
 (segment (start 170.6 70.6) (end 170.6 77.25) (width 0.2) (layer "F.Cu") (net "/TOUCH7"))
 (segment (start 170.1 70.1) (end 170.6 70.6) (width 0.2) (layer "F.Cu") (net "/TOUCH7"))
 (via (at 170.1 70.1) (size 0.6) (drill 0.3) (layers "F.Cu" "B.Cu") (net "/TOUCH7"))
 (segment (start 118.775 70.85) (end 169.35 70.85) (width 0.2) (layer "B.Cu") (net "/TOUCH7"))
 (segment (start 169.35 70.85) (end 170.1 70.1) (width 0.2) (layer "B.Cu") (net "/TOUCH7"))
 (segment (start 118.41 70.485) (end 118.775 70.85) (width 0.2) (layer "B.Cu") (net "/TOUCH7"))
 (segment (start 118.41 67.945) (end 121.262529 67.945) (width 0.2) (layer "F.Cu") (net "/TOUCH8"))
 (segment (start 121.262529 67.945) (end 128.125 74.807471) (width 0.2) (layer "F.Cu") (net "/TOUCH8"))
 (segment (start 128.125 74.807471) (end 128.125 91.775) (width 0.2) (layer "F.Cu") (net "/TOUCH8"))
 (segment (start 128.125 91.775) (end 130.6 94.25) (width 0.2) (layer "F.Cu") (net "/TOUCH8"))
 (segment (start 118.41 65.405) (end 120.405 65.405) (width 0.2) (layer "F.Cu") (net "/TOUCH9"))
 (segment (start 172.3 98.55) (end 176.6 94.25) (width 0.2) (layer "F.Cu") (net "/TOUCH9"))
 (segment (start 120.405 65.405) (end 126.95 71.95) (width 0.2) (layer "F.Cu") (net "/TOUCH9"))
 (segment (start 172.3 102.8) (end 172.3 98.55) (width 0.2) (layer "F.Cu") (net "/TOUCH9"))
 (via (at 172.3 102.8) (size 0.6) (drill 0.3) (layers "F.Cu" "B.Cu") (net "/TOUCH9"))
 (via (at 126.95 71.95) (size 0.6) (drill 0.3) (layers "F.Cu" "B.Cu") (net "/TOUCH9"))
 (segment (start 157.8 102.8) (end 172.3 102.8) (width 0.2) (layer "B.Cu") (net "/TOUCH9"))
 (segment (start 126.95 71.95) (end 157.8 102.8) (width 0.2) (layer "B.Cu") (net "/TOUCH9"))
 (segment (start 116.3 62.35) (end 116.5 62.15) (width 0.2) (layer "F.Cu") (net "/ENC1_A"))
 (segment (start 108.9 70.45) (end 110.65 68.7) (width 0.2) (layer "F.Cu") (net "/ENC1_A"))
 (segment (start 116.585 62.15) (end 118.41 60.325) (width 0.2) (layer "F.Cu") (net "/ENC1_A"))
 (segment (start 116.5 62.15) (end 116.585 62.15) (width 0.2) (layer "F.Cu") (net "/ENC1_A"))
 (via (at 108.9 70.45) (size 0.6) (drill 0.3) (layers "F.Cu" "B.Cu") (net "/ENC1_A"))
 (via (at 110.65 68.7) (size 0.6) (drill 0.3) (layers "F.Cu" "B.Cu") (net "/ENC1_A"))
 (via (at 116.3 62.35) (size 0.6) (drill 0.3) (layers "F.Cu" "B.Cu") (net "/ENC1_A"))
 (segment (start 110.65 68.7) (end 110.65 68) (width 0.2) (layer "B.Cu") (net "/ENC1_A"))
 (segment (start 108.15 70.45) (end 108.9 70.45) (width 0.2) (layer "B.Cu") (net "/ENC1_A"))
 (segment (start 110.65 68) (end 116.3 62.35) (width 0.2) (layer "B.Cu") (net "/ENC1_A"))
 (segment (start 102.365 77.975) (end 102.365 76.235) (width 0.2) (layer "B.Cu") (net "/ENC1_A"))
 (segment (start 102.365 76.235) (end 108.15 70.45) (width 0.2) (layer "B.Cu") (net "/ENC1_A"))
 (segment (start 115.5 64.05) (end 115.5 61.4) (width 0.2) (layer "F.Cu") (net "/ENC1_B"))
 (segment (start 110.45 70.65) (end 112.85 70.65) (width 0.2) (layer "F.Cu") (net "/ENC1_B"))
 (segment (start 107.3 78.04) (end 107.3 72.7) (width 0.2) (layer "F.Cu") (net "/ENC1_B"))
 (segment (start 102.365 82.975) (end 107.3 78.04) (width 0.2) (layer "F.Cu") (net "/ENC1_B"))
 (segment (start 115.5 61.4) (end 116.55 60.35) (width 0.2) (layer "F.Cu") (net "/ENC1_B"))
 (segment (start 112.85 70.65) (end 115.55 67.95) (width 0.2) (layer "F.Cu") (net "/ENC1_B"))
 (segment (start 115.55 67.95) (end 115.55 67.75) (width 0.2) (layer "F.Cu") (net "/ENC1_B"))
 (via (at 115.5 64.05) (size 0.6) (drill 0.3) (layers "F.Cu" "B.Cu") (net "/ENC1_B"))
 (via (at 115.55 67.75) (size 0.6) (drill 0.3) (layers "F.Cu" "B.Cu") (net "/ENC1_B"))
 (via (at 116.55 60.35) (size 0.6) (drill 0.3) (layers "F.Cu" "B.Cu") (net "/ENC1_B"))
 (via (at 110.45 70.65) (size 0.6) (drill 0.3) (layers "F.Cu" "B.Cu") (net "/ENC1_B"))
 (via (at 107.3 72.7) (size 0.6) (drill 0.3) (layers "F.Cu" "B.Cu") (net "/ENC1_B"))
 (segment (start 107.3 72.7) (end 108.4 72.7) (width 0.2) (layer "B.Cu") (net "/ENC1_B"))
 (segment (start 116.55 59.645) (end 118.41 57.785) (width 0.2) (layer "B.Cu") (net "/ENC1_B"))
 (segment (start 108.4 72.7) (end 110.45 70.65) (width 0.2) (layer "B.Cu") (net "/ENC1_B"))
 (segment (start 115.55 67.75) (end 115.55 64.1) (width 0.2) (layer "B.Cu") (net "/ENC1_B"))
 (segment (start 116.55 60.35) (end 116.55 59.645) (width 0.2) (layer "B.Cu") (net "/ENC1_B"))
 (segment (start 115.55 64.1) (end 115.5 64.05) (width 0.2) (layer "B.Cu") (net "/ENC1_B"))
 (segment (start 121.3 68.831) (end 121.3 71.6) (width 0.2) (layer "F.Cu") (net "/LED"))
 (segment (start 121.2 63.45) (end 121.25 63.5) (width 0.2) (layer "F.Cu") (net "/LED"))
 (segment (start 121.2 60.55) (end 121.2 63.45) (width 0.2) (layer "F.Cu") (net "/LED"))
 (segment (start 118.41 55.245) (end 121.065 57.9) (width 0.2) (layer "F.Cu") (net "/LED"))
 (segment (start 121.065 57.9) (end 121.15 57.9) (width 0.2) (layer "F.Cu") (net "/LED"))
 (via (at 121.25 63.5) (size 0.6) (drill 0.3) (layers "F.Cu" "B.Cu") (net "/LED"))
 (via (at 121.2 60.55) (size 0.6) (drill 0.3) (layers "F.Cu" "B.Cu") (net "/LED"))
 (via (at 121.3 68.831) (size 0.6) (drill 0.3) (layers "F.Cu" "B.Cu") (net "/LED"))
 (via (at 121.15 57.9) (size 0.6) (drill 0.3) (layers "F.Cu" "B.Cu") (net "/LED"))
 (via (at 121.3 71.6) (size 0.6) (drill 0.3) (layers "F.Cu" "B.Cu") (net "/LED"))
 (segment (start 121.25 68.781) (end 121.3 68.831) (width 0.2) (layer "B.Cu") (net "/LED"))
 (segment (start 125.825 73.96663) (end 125.825 74.535) (width 0.2) (layer "B.Cu") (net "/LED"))
 (segment (start 121.15 60.5) (end 121.2 60.55) (width 0.2) (layer "B.Cu") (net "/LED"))
 (segment (start 121.15 57.9) (end 121.15 60.5) (width 0.2) (layer "B.Cu") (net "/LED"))
 (segment (start 121.25 63.5) (end 121.25 68.781) (width 0.2) (layer "B.Cu") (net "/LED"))
 (segment (start 123.45837 71.6) (end 125.825 73.96663) (width 0.2) (layer "B.Cu") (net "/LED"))
 (segment (start 121.3 71.6) (end 123.45837 71.6) (width 0.2) (layer "B.Cu") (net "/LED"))
 (segment (start 95.335 49.065) (end 99.53 49.065) (width 0.2) (layer "F.Cu") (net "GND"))
 (segment (start 117.14 77.7) (end 125.4 77.7) (width 0.2) (layer "F.Cu") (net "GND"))
 (segment (start 106.15 74.97) (end 106.15 77.95) (width 0.2) (layer "F.Cu") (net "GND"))
 (segment (start 116.865 77.975) (end 117.14 77.7) (width 0.2) (layer "F.Cu") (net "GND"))
 (segment (start 99.53 49.065) (end 103.17 52.705) (width 0.2) (layer "F.Cu") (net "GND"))
 (segment (start 95.335 64.155) (end 106.15 74.97) (width 0.2) (layer "F.Cu") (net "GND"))
 (via (at 125.4 77.7) (size 0.6) (drill 0.3) (layers "F.Cu" "B.Cu") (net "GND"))
 (via (at 106.15 77.95) (size 0.6) (drill 0.3) (layers "F.Cu" "B.Cu") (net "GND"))
 (segment (start 125.4 77.7) (end 125.825 77.275) (width 0.2) (layer "B.Cu") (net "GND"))
 (segment (start 116.865 77.975) (end 113.765 74.875) (width 0.2) (layer "B.Cu") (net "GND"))
 (segment (start 95.335 64.155) (end 95.335 60.54) (width 0.2) (layer "B.Cu") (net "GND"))
 (segment (start 126.8 81.88) (end 125.825 80.905) (width 0.2) (layer "B.Cu") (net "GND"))
 (segment (start 107.965 74.875) (end 102.365 80.475) (width 0.2) (layer "B.Cu") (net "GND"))
 (segment (start 125.825 80.905) (end 126.8 79.93) (width 0.2) (layer "B.Cu") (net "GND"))
 (segment (start 106.15 77.95) (end 109.225 74.875) (width 0.2) (layer "B.Cu") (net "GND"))
 (segment (start 126.8 84.8) (end 126.8 81.88) (width 0.2) (layer "B.Cu") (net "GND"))
 (segment (start 107.975 86.075) (end 109.865 86.075) (width 0.2) (layer "B.Cu") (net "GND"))
 (segment (start 102.365 80.475) (end 102.375 80.475) (width 0.2) (layer "B.Cu") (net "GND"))
 (segment (start 125.825 77.275) (end 125.825 76.035) (width 0.2) (layer "B.Cu") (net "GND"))
 (segment (start 126.8 77.01) (end 125.825 76.035) (width 0.2) (layer "B.Cu") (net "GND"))
 (segment (start 102.375 80.475) (end 107.975 86.075) (width 0.2) (layer "B.Cu") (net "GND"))
 (segment (start 126.8 79.93) (end 126.8 77.01) (width 0.2) (layer "B.Cu") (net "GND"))
 (segment (start 109.865 74.875) (end 107.965 74.875) (width 0.2) (layer "B.Cu") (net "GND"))
 (segment (start 109.225 74.875) (end 109.865 74.875) (width 0.2) (layer "B.Cu") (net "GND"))
 (segment (start 125.825 85.775) (end 126.8 84.8) (width 0.2) (layer "B.Cu") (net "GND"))
 (segment (start 113.765 74.875) (end 109.865 74.875) (width 0.2) (layer "B.Cu") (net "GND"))
 (segment (start 95.335 60.54) (end 103.17 52.705) (width 0.2) (layer "B.Cu") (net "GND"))
 (segment (start 88.985 51.605) (end 117.31 51.605) (width 0.2) (layer "B.Cu") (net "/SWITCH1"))
 (segment (start 117.31 51.605) (end 118.41 52.705) (width 0.2) (layer "B.Cu") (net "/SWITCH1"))
 (segment (start 114.816 53.759) (end 118.41 50.165) (width 0.2) (layer "F.Cu") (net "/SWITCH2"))
 (segment (start 101.921 53.759) (end 114.816 53.759) (width 0.2) (layer "F.Cu") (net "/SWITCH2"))
 (segment (start 88.985 66.695) (end 101.921 53.759) (width 0.2) (layer "F.Cu") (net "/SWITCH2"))
 (segment (start 117 68.6) (end 117 71.35) (width 0.2) (layer "F.Cu") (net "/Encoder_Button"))
 (via (at 117 68.6) (size 0.6) (drill 0.3) (layers "F.Cu" "B.Cu") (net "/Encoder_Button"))
 (via (at 117 71.35) (size 0.6) (drill 0.3) (layers "F.Cu" "B.Cu") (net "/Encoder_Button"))
 (segment (start 118.165 81.675) (end 116.865 82.975) (width 0.2) (layer "B.Cu") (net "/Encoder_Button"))
 (segment (start 118.41 62.865) (end 117 64.275) (width 0.2) (layer "B.Cu") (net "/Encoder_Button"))
 (segment (start 117 71.35) (end 118.165 72.515) (width 0.2) (layer "B.Cu") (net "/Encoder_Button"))
 (segment (start 117 64.275) (end 117 68.6) (width 0.2) (layer "B.Cu") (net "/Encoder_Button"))
 (segment (start 118.165 72.515) (end 118.165 81.675) (width 0.2) (layer "B.Cu") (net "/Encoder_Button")))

